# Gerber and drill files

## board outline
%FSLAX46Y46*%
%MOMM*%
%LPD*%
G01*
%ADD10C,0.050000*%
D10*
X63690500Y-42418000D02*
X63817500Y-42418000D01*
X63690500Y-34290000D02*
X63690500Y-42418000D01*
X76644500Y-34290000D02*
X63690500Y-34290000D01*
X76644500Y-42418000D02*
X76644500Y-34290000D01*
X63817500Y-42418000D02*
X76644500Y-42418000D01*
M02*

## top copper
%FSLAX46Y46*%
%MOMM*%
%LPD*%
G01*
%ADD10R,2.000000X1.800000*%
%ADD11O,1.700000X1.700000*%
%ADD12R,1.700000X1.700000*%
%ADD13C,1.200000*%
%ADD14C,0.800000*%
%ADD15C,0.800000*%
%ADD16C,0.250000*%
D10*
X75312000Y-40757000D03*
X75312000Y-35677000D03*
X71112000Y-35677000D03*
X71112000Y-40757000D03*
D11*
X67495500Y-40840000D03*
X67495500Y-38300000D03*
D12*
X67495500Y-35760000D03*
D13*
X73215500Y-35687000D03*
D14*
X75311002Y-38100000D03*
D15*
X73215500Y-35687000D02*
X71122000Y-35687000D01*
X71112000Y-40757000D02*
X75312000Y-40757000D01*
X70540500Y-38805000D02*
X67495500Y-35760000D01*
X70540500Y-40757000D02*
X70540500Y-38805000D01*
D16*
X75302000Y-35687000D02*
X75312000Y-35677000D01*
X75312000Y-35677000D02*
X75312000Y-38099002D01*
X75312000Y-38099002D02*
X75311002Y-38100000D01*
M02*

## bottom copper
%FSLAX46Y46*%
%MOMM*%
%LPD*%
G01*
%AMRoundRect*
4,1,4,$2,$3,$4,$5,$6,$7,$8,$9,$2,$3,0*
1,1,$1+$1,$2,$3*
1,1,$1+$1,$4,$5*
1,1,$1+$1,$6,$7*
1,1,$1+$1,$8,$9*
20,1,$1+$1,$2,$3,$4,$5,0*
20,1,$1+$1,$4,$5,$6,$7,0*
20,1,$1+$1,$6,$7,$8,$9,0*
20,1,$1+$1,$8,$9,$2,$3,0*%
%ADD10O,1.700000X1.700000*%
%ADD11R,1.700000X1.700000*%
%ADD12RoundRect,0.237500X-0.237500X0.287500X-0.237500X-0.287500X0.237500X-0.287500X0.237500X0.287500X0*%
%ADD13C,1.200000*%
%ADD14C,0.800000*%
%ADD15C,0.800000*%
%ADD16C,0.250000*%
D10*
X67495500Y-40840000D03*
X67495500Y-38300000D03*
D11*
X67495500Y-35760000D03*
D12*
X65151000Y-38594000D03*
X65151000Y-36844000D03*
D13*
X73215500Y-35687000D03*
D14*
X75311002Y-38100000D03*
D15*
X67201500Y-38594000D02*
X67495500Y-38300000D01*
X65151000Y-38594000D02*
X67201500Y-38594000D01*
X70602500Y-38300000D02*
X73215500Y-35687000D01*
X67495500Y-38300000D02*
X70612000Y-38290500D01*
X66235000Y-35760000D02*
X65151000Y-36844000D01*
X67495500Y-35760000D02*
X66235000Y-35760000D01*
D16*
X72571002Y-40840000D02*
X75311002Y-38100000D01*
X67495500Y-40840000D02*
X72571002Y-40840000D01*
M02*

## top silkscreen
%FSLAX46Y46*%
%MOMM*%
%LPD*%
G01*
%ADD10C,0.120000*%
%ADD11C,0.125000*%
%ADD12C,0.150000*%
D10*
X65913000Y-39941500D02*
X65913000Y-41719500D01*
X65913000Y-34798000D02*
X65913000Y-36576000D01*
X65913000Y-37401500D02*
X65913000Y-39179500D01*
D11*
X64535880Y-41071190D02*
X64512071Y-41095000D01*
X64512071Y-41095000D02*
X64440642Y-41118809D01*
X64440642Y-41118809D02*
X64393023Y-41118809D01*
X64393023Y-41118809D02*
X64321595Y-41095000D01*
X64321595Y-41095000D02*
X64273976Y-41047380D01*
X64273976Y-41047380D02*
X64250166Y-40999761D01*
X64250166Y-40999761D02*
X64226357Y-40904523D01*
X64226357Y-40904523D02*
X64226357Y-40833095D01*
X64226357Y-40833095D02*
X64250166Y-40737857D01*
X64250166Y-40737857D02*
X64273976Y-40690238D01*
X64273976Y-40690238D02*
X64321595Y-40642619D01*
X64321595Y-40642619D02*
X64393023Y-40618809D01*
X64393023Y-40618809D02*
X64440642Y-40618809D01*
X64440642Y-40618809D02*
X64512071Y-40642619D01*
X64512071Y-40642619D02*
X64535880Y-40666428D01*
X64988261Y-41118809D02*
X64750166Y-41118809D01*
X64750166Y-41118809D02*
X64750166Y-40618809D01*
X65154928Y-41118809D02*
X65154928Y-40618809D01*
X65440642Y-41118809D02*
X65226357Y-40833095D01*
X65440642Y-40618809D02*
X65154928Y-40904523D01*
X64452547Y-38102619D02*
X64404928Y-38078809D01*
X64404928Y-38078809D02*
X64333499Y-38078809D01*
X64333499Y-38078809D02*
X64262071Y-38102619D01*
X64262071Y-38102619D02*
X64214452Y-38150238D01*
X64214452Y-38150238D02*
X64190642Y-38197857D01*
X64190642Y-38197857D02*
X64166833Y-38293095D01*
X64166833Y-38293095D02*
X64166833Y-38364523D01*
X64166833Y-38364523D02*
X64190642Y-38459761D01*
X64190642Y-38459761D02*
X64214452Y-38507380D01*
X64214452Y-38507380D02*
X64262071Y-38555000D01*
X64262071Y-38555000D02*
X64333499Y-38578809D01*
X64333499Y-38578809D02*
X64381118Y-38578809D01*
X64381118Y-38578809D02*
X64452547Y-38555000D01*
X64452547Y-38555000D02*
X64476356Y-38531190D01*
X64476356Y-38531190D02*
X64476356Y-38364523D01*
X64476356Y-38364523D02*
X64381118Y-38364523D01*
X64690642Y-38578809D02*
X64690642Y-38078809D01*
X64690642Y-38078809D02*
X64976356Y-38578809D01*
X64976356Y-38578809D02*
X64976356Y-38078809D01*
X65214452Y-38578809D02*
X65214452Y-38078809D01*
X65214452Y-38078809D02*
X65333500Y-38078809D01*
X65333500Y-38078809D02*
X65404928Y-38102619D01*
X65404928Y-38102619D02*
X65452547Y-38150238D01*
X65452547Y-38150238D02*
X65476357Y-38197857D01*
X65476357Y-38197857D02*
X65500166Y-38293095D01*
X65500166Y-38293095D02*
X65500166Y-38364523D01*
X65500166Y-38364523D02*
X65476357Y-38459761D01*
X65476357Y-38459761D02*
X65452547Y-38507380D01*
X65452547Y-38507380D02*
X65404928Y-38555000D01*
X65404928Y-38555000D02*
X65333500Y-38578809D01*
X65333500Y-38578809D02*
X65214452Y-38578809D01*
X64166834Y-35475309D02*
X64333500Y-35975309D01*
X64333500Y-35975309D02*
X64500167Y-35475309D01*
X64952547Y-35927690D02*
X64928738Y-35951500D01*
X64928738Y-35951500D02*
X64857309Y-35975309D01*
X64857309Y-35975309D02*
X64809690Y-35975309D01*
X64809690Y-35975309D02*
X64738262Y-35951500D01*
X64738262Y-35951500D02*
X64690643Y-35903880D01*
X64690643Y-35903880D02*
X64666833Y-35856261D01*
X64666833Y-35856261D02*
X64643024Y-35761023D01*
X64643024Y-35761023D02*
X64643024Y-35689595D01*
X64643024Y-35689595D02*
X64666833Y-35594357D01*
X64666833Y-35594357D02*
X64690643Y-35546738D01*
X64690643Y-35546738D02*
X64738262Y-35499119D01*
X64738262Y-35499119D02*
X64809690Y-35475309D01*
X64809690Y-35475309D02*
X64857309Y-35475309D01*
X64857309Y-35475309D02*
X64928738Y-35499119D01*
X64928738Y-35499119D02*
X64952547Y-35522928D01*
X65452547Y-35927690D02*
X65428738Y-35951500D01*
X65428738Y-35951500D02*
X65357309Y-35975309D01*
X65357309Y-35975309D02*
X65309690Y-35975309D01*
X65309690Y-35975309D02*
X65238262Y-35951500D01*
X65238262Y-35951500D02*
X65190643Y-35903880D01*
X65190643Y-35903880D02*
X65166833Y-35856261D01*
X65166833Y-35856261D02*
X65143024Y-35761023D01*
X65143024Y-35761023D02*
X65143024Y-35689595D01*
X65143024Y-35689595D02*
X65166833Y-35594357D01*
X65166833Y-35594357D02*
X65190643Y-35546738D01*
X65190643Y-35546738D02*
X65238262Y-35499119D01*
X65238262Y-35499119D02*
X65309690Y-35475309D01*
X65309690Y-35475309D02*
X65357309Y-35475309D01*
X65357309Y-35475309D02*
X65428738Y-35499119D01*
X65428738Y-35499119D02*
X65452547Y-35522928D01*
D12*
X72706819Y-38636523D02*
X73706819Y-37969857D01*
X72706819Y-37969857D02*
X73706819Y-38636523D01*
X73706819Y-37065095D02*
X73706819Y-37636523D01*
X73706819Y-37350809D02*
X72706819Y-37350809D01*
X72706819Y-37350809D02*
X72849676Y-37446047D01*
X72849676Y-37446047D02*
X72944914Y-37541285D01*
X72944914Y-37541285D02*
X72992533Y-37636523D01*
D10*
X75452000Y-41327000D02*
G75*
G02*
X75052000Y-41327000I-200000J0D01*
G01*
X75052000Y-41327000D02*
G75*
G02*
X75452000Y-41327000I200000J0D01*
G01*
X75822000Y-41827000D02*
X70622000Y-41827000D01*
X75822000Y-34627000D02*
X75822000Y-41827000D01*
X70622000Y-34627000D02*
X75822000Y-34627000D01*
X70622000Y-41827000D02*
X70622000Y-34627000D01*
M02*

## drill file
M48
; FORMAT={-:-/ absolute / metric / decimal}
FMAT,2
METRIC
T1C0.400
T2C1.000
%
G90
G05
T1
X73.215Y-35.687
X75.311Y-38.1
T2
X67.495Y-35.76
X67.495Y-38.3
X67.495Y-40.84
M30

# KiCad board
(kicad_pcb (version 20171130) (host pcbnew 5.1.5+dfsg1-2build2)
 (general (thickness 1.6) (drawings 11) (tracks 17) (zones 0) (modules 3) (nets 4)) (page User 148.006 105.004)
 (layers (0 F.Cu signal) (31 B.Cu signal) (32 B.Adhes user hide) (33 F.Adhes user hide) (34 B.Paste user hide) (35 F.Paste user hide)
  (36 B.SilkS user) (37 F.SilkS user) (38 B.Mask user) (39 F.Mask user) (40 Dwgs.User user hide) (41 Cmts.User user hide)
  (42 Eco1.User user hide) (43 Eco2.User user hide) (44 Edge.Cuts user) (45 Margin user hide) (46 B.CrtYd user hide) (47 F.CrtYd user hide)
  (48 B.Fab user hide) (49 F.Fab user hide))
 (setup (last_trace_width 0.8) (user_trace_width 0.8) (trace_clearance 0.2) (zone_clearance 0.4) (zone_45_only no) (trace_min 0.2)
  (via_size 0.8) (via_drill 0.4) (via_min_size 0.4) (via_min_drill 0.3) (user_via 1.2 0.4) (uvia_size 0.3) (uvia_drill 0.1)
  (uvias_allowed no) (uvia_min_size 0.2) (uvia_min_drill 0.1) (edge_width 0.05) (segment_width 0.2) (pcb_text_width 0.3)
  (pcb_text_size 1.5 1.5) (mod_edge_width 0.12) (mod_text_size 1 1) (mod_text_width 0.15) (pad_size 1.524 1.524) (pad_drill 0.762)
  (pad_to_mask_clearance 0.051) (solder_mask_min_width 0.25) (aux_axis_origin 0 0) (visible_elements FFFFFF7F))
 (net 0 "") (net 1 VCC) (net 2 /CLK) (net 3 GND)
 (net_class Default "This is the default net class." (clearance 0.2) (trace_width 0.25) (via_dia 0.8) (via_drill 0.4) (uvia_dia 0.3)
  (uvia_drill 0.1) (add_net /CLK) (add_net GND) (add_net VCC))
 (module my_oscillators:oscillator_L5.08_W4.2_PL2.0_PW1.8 (layer F.Cu) (at 73.152 38.227 90)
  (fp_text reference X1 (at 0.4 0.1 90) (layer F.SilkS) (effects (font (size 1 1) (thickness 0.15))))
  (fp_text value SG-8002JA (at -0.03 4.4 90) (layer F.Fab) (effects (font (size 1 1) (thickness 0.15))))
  (fp_circle (center -3.1 2.1) (end -2.9 2.1) (layer F.SilkS) (width 0.12))
  (fp_line (start -3.6 2.67) (end -3.6 -2.53) (layer F.SilkS) (width 0.12))
  (fp_line (start 3.6 2.67) (end -3.6 2.67) (layer F.SilkS) (width 0.12))
  (fp_line (start 3.6 -2.53) (end 3.6 2.67) (layer F.SilkS) (width 0.12))
  (fp_line (start -3.6 -2.53) (end 3.6 -2.53) (layer F.SilkS) (width 0.12))
  (pad 4 smd rect (at -2.53 2.16 90) (size 1.8 2) (layers F.Cu F.Paste F.Mask) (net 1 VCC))
  (pad 3 smd rect (at 2.55 2.16 90) (size 1.8 2) (layers F.Cu F.Paste F.Mask) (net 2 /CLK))
  (pad 2 smd rect (at 2.55 -2.04 90) (size 1.8 2) (layers F.Cu F.Paste F.Mask) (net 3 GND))
  (pad 1 smd rect (at -2.53 -2.04 90) (size 1.8 2) (layers F.Cu F.Paste F.Mask) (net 1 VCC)))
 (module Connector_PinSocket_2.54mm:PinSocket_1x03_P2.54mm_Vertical (layer B.Cu) (at 67.4955 35.76 180)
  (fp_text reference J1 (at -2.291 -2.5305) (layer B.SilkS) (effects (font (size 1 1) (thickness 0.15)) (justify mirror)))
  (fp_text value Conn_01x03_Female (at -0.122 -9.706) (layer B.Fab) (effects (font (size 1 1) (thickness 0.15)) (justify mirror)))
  (pad 3 thru_hole oval (at 0 -5.08 180) (size 1.7 1.7) (drill 1) (layers *.Cu *.Mask) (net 2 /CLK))
  (pad 2 thru_hole oval (at 0 -2.54 180) (size 1.7 1.7) (drill 1) (layers *.Cu *.Mask) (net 3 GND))
  (pad 1 thru_hole rect (at 0 0 180) (size 1.7 1.7) (drill 1) (layers *.Cu *.Mask) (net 1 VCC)))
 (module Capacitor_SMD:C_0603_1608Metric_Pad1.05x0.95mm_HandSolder (layer B.Cu) (at 65.151 37.719 270)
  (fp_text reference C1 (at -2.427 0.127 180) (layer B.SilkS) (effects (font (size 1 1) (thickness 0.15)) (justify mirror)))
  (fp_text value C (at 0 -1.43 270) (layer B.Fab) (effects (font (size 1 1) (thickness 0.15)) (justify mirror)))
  (pad 2 smd roundrect (at 0.875 0 270) (size 1.05 0.95) (layers B.Cu B.Paste B.Mask) (roundrect_rratio 0.25) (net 3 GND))
  (pad 1 smd roundrect (at -0.875 0 270) (size 1.05 0.95) (layers B.Cu B.Paste B.Mask) (roundrect_rratio 0.25) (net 1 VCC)))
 (gr_line (start 65.913 39.9415) (end 65.913 41.7195) (layer F.SilkS) (width 0.12))
 (gr_line (start 65.913 34.798) (end 65.913 36.576) (layer F.SilkS) (width 0.12))
 (gr_line (start 65.913 37.4015) (end 65.913 39.1795) (layer F.SilkS) (width 0.12))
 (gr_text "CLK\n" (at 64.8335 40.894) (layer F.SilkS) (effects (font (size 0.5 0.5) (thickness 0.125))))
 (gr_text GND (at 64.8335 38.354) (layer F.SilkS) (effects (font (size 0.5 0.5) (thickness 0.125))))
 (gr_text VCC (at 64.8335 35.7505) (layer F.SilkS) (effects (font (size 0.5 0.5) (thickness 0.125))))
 (gr_line (start 63.6905 42.418) (end 63.8175 42.418) (layer Edge.Cuts) (width 0.05))
 (gr_line (start 63.6905 34.29) (end 63.6905 42.418) (layer Edge.Cuts) (width 0.05))
 (gr_line (start 76.6445 34.29) (end 63.6905 34.29) (layer Edge.Cuts) (width 0.05))
 (gr_line (start 76.6445 42.418) (end 76.6445 34.29) (layer Edge.Cuts) (width 0.05))
 (gr_line (start 63.8175 42.418) (end 76.6445 42.418) (layer Edge.Cuts) (width 0.05))
 (via (at 73.2155 35.687) (size 1.2) (drill 0.4) (layers F.Cu B.Cu) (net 3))
 (segment (start 73.2155 35.687) (end 71.122 35.687) (width 0.8) (layer F.Cu) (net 3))
 (segment (start 67.2015 38.594) (end 67.4955 38.3) (width 0.8) (layer B.Cu) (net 3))
 (segment (start 65.151 38.594) (end 67.2015 38.594) (width 0.8) (layer B.Cu) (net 3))
 (segment (start 70.6025 38.3) (end 73.2155 35.687) (width 0.8) (layer B.Cu) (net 3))
 (segment (start 67.4955 38.3) (end 70.612 38.2905) (width 0.8) (layer B.Cu) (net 3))
 (segment (start 71.112 40.757) (end 75.312 40.757) (width 0.8) (layer F.Cu) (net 1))
 (segment (start 70.5405 38.805) (end 67.4955 35.76) (width 0.8) (layer F.Cu) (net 1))
 (segment (start 70.5405 40.757) (end 70.5405 38.805) (width 0.8) (layer F.Cu) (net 1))
 (segment (start 66.235 35.76) (end 65.151 36.844) (width 0.8) (layer B.Cu) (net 1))
 (segment (start 67.4955 35.76) (end 66.235 35.76) (width 0.8) (layer B.Cu) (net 1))
 (segment (start 75.302 35.687) (end 75.312 35.677) (width 0.25) (layer F.Cu) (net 2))
 (via (at 75.311002 38.1) (size 0.8) (drill 0.4) (layers F.Cu B.Cu) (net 2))
 (segment (start 75.312 35.677) (end 75.312 38.099002) (width 0.25) (layer F.Cu) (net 2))
 (segment (start 75.312 38.099002) (end 75.311002 38.1) (width 0.25) (layer F.Cu) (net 2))
 (segment (start 72.571002 40.84) (end 75.311002 38.1) (width 0.25) (layer B.Cu) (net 2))
 (segment (start 67.4955 40.84) (end 72.571002 40.84) (width 0.25) (layer B.Cu) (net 2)))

